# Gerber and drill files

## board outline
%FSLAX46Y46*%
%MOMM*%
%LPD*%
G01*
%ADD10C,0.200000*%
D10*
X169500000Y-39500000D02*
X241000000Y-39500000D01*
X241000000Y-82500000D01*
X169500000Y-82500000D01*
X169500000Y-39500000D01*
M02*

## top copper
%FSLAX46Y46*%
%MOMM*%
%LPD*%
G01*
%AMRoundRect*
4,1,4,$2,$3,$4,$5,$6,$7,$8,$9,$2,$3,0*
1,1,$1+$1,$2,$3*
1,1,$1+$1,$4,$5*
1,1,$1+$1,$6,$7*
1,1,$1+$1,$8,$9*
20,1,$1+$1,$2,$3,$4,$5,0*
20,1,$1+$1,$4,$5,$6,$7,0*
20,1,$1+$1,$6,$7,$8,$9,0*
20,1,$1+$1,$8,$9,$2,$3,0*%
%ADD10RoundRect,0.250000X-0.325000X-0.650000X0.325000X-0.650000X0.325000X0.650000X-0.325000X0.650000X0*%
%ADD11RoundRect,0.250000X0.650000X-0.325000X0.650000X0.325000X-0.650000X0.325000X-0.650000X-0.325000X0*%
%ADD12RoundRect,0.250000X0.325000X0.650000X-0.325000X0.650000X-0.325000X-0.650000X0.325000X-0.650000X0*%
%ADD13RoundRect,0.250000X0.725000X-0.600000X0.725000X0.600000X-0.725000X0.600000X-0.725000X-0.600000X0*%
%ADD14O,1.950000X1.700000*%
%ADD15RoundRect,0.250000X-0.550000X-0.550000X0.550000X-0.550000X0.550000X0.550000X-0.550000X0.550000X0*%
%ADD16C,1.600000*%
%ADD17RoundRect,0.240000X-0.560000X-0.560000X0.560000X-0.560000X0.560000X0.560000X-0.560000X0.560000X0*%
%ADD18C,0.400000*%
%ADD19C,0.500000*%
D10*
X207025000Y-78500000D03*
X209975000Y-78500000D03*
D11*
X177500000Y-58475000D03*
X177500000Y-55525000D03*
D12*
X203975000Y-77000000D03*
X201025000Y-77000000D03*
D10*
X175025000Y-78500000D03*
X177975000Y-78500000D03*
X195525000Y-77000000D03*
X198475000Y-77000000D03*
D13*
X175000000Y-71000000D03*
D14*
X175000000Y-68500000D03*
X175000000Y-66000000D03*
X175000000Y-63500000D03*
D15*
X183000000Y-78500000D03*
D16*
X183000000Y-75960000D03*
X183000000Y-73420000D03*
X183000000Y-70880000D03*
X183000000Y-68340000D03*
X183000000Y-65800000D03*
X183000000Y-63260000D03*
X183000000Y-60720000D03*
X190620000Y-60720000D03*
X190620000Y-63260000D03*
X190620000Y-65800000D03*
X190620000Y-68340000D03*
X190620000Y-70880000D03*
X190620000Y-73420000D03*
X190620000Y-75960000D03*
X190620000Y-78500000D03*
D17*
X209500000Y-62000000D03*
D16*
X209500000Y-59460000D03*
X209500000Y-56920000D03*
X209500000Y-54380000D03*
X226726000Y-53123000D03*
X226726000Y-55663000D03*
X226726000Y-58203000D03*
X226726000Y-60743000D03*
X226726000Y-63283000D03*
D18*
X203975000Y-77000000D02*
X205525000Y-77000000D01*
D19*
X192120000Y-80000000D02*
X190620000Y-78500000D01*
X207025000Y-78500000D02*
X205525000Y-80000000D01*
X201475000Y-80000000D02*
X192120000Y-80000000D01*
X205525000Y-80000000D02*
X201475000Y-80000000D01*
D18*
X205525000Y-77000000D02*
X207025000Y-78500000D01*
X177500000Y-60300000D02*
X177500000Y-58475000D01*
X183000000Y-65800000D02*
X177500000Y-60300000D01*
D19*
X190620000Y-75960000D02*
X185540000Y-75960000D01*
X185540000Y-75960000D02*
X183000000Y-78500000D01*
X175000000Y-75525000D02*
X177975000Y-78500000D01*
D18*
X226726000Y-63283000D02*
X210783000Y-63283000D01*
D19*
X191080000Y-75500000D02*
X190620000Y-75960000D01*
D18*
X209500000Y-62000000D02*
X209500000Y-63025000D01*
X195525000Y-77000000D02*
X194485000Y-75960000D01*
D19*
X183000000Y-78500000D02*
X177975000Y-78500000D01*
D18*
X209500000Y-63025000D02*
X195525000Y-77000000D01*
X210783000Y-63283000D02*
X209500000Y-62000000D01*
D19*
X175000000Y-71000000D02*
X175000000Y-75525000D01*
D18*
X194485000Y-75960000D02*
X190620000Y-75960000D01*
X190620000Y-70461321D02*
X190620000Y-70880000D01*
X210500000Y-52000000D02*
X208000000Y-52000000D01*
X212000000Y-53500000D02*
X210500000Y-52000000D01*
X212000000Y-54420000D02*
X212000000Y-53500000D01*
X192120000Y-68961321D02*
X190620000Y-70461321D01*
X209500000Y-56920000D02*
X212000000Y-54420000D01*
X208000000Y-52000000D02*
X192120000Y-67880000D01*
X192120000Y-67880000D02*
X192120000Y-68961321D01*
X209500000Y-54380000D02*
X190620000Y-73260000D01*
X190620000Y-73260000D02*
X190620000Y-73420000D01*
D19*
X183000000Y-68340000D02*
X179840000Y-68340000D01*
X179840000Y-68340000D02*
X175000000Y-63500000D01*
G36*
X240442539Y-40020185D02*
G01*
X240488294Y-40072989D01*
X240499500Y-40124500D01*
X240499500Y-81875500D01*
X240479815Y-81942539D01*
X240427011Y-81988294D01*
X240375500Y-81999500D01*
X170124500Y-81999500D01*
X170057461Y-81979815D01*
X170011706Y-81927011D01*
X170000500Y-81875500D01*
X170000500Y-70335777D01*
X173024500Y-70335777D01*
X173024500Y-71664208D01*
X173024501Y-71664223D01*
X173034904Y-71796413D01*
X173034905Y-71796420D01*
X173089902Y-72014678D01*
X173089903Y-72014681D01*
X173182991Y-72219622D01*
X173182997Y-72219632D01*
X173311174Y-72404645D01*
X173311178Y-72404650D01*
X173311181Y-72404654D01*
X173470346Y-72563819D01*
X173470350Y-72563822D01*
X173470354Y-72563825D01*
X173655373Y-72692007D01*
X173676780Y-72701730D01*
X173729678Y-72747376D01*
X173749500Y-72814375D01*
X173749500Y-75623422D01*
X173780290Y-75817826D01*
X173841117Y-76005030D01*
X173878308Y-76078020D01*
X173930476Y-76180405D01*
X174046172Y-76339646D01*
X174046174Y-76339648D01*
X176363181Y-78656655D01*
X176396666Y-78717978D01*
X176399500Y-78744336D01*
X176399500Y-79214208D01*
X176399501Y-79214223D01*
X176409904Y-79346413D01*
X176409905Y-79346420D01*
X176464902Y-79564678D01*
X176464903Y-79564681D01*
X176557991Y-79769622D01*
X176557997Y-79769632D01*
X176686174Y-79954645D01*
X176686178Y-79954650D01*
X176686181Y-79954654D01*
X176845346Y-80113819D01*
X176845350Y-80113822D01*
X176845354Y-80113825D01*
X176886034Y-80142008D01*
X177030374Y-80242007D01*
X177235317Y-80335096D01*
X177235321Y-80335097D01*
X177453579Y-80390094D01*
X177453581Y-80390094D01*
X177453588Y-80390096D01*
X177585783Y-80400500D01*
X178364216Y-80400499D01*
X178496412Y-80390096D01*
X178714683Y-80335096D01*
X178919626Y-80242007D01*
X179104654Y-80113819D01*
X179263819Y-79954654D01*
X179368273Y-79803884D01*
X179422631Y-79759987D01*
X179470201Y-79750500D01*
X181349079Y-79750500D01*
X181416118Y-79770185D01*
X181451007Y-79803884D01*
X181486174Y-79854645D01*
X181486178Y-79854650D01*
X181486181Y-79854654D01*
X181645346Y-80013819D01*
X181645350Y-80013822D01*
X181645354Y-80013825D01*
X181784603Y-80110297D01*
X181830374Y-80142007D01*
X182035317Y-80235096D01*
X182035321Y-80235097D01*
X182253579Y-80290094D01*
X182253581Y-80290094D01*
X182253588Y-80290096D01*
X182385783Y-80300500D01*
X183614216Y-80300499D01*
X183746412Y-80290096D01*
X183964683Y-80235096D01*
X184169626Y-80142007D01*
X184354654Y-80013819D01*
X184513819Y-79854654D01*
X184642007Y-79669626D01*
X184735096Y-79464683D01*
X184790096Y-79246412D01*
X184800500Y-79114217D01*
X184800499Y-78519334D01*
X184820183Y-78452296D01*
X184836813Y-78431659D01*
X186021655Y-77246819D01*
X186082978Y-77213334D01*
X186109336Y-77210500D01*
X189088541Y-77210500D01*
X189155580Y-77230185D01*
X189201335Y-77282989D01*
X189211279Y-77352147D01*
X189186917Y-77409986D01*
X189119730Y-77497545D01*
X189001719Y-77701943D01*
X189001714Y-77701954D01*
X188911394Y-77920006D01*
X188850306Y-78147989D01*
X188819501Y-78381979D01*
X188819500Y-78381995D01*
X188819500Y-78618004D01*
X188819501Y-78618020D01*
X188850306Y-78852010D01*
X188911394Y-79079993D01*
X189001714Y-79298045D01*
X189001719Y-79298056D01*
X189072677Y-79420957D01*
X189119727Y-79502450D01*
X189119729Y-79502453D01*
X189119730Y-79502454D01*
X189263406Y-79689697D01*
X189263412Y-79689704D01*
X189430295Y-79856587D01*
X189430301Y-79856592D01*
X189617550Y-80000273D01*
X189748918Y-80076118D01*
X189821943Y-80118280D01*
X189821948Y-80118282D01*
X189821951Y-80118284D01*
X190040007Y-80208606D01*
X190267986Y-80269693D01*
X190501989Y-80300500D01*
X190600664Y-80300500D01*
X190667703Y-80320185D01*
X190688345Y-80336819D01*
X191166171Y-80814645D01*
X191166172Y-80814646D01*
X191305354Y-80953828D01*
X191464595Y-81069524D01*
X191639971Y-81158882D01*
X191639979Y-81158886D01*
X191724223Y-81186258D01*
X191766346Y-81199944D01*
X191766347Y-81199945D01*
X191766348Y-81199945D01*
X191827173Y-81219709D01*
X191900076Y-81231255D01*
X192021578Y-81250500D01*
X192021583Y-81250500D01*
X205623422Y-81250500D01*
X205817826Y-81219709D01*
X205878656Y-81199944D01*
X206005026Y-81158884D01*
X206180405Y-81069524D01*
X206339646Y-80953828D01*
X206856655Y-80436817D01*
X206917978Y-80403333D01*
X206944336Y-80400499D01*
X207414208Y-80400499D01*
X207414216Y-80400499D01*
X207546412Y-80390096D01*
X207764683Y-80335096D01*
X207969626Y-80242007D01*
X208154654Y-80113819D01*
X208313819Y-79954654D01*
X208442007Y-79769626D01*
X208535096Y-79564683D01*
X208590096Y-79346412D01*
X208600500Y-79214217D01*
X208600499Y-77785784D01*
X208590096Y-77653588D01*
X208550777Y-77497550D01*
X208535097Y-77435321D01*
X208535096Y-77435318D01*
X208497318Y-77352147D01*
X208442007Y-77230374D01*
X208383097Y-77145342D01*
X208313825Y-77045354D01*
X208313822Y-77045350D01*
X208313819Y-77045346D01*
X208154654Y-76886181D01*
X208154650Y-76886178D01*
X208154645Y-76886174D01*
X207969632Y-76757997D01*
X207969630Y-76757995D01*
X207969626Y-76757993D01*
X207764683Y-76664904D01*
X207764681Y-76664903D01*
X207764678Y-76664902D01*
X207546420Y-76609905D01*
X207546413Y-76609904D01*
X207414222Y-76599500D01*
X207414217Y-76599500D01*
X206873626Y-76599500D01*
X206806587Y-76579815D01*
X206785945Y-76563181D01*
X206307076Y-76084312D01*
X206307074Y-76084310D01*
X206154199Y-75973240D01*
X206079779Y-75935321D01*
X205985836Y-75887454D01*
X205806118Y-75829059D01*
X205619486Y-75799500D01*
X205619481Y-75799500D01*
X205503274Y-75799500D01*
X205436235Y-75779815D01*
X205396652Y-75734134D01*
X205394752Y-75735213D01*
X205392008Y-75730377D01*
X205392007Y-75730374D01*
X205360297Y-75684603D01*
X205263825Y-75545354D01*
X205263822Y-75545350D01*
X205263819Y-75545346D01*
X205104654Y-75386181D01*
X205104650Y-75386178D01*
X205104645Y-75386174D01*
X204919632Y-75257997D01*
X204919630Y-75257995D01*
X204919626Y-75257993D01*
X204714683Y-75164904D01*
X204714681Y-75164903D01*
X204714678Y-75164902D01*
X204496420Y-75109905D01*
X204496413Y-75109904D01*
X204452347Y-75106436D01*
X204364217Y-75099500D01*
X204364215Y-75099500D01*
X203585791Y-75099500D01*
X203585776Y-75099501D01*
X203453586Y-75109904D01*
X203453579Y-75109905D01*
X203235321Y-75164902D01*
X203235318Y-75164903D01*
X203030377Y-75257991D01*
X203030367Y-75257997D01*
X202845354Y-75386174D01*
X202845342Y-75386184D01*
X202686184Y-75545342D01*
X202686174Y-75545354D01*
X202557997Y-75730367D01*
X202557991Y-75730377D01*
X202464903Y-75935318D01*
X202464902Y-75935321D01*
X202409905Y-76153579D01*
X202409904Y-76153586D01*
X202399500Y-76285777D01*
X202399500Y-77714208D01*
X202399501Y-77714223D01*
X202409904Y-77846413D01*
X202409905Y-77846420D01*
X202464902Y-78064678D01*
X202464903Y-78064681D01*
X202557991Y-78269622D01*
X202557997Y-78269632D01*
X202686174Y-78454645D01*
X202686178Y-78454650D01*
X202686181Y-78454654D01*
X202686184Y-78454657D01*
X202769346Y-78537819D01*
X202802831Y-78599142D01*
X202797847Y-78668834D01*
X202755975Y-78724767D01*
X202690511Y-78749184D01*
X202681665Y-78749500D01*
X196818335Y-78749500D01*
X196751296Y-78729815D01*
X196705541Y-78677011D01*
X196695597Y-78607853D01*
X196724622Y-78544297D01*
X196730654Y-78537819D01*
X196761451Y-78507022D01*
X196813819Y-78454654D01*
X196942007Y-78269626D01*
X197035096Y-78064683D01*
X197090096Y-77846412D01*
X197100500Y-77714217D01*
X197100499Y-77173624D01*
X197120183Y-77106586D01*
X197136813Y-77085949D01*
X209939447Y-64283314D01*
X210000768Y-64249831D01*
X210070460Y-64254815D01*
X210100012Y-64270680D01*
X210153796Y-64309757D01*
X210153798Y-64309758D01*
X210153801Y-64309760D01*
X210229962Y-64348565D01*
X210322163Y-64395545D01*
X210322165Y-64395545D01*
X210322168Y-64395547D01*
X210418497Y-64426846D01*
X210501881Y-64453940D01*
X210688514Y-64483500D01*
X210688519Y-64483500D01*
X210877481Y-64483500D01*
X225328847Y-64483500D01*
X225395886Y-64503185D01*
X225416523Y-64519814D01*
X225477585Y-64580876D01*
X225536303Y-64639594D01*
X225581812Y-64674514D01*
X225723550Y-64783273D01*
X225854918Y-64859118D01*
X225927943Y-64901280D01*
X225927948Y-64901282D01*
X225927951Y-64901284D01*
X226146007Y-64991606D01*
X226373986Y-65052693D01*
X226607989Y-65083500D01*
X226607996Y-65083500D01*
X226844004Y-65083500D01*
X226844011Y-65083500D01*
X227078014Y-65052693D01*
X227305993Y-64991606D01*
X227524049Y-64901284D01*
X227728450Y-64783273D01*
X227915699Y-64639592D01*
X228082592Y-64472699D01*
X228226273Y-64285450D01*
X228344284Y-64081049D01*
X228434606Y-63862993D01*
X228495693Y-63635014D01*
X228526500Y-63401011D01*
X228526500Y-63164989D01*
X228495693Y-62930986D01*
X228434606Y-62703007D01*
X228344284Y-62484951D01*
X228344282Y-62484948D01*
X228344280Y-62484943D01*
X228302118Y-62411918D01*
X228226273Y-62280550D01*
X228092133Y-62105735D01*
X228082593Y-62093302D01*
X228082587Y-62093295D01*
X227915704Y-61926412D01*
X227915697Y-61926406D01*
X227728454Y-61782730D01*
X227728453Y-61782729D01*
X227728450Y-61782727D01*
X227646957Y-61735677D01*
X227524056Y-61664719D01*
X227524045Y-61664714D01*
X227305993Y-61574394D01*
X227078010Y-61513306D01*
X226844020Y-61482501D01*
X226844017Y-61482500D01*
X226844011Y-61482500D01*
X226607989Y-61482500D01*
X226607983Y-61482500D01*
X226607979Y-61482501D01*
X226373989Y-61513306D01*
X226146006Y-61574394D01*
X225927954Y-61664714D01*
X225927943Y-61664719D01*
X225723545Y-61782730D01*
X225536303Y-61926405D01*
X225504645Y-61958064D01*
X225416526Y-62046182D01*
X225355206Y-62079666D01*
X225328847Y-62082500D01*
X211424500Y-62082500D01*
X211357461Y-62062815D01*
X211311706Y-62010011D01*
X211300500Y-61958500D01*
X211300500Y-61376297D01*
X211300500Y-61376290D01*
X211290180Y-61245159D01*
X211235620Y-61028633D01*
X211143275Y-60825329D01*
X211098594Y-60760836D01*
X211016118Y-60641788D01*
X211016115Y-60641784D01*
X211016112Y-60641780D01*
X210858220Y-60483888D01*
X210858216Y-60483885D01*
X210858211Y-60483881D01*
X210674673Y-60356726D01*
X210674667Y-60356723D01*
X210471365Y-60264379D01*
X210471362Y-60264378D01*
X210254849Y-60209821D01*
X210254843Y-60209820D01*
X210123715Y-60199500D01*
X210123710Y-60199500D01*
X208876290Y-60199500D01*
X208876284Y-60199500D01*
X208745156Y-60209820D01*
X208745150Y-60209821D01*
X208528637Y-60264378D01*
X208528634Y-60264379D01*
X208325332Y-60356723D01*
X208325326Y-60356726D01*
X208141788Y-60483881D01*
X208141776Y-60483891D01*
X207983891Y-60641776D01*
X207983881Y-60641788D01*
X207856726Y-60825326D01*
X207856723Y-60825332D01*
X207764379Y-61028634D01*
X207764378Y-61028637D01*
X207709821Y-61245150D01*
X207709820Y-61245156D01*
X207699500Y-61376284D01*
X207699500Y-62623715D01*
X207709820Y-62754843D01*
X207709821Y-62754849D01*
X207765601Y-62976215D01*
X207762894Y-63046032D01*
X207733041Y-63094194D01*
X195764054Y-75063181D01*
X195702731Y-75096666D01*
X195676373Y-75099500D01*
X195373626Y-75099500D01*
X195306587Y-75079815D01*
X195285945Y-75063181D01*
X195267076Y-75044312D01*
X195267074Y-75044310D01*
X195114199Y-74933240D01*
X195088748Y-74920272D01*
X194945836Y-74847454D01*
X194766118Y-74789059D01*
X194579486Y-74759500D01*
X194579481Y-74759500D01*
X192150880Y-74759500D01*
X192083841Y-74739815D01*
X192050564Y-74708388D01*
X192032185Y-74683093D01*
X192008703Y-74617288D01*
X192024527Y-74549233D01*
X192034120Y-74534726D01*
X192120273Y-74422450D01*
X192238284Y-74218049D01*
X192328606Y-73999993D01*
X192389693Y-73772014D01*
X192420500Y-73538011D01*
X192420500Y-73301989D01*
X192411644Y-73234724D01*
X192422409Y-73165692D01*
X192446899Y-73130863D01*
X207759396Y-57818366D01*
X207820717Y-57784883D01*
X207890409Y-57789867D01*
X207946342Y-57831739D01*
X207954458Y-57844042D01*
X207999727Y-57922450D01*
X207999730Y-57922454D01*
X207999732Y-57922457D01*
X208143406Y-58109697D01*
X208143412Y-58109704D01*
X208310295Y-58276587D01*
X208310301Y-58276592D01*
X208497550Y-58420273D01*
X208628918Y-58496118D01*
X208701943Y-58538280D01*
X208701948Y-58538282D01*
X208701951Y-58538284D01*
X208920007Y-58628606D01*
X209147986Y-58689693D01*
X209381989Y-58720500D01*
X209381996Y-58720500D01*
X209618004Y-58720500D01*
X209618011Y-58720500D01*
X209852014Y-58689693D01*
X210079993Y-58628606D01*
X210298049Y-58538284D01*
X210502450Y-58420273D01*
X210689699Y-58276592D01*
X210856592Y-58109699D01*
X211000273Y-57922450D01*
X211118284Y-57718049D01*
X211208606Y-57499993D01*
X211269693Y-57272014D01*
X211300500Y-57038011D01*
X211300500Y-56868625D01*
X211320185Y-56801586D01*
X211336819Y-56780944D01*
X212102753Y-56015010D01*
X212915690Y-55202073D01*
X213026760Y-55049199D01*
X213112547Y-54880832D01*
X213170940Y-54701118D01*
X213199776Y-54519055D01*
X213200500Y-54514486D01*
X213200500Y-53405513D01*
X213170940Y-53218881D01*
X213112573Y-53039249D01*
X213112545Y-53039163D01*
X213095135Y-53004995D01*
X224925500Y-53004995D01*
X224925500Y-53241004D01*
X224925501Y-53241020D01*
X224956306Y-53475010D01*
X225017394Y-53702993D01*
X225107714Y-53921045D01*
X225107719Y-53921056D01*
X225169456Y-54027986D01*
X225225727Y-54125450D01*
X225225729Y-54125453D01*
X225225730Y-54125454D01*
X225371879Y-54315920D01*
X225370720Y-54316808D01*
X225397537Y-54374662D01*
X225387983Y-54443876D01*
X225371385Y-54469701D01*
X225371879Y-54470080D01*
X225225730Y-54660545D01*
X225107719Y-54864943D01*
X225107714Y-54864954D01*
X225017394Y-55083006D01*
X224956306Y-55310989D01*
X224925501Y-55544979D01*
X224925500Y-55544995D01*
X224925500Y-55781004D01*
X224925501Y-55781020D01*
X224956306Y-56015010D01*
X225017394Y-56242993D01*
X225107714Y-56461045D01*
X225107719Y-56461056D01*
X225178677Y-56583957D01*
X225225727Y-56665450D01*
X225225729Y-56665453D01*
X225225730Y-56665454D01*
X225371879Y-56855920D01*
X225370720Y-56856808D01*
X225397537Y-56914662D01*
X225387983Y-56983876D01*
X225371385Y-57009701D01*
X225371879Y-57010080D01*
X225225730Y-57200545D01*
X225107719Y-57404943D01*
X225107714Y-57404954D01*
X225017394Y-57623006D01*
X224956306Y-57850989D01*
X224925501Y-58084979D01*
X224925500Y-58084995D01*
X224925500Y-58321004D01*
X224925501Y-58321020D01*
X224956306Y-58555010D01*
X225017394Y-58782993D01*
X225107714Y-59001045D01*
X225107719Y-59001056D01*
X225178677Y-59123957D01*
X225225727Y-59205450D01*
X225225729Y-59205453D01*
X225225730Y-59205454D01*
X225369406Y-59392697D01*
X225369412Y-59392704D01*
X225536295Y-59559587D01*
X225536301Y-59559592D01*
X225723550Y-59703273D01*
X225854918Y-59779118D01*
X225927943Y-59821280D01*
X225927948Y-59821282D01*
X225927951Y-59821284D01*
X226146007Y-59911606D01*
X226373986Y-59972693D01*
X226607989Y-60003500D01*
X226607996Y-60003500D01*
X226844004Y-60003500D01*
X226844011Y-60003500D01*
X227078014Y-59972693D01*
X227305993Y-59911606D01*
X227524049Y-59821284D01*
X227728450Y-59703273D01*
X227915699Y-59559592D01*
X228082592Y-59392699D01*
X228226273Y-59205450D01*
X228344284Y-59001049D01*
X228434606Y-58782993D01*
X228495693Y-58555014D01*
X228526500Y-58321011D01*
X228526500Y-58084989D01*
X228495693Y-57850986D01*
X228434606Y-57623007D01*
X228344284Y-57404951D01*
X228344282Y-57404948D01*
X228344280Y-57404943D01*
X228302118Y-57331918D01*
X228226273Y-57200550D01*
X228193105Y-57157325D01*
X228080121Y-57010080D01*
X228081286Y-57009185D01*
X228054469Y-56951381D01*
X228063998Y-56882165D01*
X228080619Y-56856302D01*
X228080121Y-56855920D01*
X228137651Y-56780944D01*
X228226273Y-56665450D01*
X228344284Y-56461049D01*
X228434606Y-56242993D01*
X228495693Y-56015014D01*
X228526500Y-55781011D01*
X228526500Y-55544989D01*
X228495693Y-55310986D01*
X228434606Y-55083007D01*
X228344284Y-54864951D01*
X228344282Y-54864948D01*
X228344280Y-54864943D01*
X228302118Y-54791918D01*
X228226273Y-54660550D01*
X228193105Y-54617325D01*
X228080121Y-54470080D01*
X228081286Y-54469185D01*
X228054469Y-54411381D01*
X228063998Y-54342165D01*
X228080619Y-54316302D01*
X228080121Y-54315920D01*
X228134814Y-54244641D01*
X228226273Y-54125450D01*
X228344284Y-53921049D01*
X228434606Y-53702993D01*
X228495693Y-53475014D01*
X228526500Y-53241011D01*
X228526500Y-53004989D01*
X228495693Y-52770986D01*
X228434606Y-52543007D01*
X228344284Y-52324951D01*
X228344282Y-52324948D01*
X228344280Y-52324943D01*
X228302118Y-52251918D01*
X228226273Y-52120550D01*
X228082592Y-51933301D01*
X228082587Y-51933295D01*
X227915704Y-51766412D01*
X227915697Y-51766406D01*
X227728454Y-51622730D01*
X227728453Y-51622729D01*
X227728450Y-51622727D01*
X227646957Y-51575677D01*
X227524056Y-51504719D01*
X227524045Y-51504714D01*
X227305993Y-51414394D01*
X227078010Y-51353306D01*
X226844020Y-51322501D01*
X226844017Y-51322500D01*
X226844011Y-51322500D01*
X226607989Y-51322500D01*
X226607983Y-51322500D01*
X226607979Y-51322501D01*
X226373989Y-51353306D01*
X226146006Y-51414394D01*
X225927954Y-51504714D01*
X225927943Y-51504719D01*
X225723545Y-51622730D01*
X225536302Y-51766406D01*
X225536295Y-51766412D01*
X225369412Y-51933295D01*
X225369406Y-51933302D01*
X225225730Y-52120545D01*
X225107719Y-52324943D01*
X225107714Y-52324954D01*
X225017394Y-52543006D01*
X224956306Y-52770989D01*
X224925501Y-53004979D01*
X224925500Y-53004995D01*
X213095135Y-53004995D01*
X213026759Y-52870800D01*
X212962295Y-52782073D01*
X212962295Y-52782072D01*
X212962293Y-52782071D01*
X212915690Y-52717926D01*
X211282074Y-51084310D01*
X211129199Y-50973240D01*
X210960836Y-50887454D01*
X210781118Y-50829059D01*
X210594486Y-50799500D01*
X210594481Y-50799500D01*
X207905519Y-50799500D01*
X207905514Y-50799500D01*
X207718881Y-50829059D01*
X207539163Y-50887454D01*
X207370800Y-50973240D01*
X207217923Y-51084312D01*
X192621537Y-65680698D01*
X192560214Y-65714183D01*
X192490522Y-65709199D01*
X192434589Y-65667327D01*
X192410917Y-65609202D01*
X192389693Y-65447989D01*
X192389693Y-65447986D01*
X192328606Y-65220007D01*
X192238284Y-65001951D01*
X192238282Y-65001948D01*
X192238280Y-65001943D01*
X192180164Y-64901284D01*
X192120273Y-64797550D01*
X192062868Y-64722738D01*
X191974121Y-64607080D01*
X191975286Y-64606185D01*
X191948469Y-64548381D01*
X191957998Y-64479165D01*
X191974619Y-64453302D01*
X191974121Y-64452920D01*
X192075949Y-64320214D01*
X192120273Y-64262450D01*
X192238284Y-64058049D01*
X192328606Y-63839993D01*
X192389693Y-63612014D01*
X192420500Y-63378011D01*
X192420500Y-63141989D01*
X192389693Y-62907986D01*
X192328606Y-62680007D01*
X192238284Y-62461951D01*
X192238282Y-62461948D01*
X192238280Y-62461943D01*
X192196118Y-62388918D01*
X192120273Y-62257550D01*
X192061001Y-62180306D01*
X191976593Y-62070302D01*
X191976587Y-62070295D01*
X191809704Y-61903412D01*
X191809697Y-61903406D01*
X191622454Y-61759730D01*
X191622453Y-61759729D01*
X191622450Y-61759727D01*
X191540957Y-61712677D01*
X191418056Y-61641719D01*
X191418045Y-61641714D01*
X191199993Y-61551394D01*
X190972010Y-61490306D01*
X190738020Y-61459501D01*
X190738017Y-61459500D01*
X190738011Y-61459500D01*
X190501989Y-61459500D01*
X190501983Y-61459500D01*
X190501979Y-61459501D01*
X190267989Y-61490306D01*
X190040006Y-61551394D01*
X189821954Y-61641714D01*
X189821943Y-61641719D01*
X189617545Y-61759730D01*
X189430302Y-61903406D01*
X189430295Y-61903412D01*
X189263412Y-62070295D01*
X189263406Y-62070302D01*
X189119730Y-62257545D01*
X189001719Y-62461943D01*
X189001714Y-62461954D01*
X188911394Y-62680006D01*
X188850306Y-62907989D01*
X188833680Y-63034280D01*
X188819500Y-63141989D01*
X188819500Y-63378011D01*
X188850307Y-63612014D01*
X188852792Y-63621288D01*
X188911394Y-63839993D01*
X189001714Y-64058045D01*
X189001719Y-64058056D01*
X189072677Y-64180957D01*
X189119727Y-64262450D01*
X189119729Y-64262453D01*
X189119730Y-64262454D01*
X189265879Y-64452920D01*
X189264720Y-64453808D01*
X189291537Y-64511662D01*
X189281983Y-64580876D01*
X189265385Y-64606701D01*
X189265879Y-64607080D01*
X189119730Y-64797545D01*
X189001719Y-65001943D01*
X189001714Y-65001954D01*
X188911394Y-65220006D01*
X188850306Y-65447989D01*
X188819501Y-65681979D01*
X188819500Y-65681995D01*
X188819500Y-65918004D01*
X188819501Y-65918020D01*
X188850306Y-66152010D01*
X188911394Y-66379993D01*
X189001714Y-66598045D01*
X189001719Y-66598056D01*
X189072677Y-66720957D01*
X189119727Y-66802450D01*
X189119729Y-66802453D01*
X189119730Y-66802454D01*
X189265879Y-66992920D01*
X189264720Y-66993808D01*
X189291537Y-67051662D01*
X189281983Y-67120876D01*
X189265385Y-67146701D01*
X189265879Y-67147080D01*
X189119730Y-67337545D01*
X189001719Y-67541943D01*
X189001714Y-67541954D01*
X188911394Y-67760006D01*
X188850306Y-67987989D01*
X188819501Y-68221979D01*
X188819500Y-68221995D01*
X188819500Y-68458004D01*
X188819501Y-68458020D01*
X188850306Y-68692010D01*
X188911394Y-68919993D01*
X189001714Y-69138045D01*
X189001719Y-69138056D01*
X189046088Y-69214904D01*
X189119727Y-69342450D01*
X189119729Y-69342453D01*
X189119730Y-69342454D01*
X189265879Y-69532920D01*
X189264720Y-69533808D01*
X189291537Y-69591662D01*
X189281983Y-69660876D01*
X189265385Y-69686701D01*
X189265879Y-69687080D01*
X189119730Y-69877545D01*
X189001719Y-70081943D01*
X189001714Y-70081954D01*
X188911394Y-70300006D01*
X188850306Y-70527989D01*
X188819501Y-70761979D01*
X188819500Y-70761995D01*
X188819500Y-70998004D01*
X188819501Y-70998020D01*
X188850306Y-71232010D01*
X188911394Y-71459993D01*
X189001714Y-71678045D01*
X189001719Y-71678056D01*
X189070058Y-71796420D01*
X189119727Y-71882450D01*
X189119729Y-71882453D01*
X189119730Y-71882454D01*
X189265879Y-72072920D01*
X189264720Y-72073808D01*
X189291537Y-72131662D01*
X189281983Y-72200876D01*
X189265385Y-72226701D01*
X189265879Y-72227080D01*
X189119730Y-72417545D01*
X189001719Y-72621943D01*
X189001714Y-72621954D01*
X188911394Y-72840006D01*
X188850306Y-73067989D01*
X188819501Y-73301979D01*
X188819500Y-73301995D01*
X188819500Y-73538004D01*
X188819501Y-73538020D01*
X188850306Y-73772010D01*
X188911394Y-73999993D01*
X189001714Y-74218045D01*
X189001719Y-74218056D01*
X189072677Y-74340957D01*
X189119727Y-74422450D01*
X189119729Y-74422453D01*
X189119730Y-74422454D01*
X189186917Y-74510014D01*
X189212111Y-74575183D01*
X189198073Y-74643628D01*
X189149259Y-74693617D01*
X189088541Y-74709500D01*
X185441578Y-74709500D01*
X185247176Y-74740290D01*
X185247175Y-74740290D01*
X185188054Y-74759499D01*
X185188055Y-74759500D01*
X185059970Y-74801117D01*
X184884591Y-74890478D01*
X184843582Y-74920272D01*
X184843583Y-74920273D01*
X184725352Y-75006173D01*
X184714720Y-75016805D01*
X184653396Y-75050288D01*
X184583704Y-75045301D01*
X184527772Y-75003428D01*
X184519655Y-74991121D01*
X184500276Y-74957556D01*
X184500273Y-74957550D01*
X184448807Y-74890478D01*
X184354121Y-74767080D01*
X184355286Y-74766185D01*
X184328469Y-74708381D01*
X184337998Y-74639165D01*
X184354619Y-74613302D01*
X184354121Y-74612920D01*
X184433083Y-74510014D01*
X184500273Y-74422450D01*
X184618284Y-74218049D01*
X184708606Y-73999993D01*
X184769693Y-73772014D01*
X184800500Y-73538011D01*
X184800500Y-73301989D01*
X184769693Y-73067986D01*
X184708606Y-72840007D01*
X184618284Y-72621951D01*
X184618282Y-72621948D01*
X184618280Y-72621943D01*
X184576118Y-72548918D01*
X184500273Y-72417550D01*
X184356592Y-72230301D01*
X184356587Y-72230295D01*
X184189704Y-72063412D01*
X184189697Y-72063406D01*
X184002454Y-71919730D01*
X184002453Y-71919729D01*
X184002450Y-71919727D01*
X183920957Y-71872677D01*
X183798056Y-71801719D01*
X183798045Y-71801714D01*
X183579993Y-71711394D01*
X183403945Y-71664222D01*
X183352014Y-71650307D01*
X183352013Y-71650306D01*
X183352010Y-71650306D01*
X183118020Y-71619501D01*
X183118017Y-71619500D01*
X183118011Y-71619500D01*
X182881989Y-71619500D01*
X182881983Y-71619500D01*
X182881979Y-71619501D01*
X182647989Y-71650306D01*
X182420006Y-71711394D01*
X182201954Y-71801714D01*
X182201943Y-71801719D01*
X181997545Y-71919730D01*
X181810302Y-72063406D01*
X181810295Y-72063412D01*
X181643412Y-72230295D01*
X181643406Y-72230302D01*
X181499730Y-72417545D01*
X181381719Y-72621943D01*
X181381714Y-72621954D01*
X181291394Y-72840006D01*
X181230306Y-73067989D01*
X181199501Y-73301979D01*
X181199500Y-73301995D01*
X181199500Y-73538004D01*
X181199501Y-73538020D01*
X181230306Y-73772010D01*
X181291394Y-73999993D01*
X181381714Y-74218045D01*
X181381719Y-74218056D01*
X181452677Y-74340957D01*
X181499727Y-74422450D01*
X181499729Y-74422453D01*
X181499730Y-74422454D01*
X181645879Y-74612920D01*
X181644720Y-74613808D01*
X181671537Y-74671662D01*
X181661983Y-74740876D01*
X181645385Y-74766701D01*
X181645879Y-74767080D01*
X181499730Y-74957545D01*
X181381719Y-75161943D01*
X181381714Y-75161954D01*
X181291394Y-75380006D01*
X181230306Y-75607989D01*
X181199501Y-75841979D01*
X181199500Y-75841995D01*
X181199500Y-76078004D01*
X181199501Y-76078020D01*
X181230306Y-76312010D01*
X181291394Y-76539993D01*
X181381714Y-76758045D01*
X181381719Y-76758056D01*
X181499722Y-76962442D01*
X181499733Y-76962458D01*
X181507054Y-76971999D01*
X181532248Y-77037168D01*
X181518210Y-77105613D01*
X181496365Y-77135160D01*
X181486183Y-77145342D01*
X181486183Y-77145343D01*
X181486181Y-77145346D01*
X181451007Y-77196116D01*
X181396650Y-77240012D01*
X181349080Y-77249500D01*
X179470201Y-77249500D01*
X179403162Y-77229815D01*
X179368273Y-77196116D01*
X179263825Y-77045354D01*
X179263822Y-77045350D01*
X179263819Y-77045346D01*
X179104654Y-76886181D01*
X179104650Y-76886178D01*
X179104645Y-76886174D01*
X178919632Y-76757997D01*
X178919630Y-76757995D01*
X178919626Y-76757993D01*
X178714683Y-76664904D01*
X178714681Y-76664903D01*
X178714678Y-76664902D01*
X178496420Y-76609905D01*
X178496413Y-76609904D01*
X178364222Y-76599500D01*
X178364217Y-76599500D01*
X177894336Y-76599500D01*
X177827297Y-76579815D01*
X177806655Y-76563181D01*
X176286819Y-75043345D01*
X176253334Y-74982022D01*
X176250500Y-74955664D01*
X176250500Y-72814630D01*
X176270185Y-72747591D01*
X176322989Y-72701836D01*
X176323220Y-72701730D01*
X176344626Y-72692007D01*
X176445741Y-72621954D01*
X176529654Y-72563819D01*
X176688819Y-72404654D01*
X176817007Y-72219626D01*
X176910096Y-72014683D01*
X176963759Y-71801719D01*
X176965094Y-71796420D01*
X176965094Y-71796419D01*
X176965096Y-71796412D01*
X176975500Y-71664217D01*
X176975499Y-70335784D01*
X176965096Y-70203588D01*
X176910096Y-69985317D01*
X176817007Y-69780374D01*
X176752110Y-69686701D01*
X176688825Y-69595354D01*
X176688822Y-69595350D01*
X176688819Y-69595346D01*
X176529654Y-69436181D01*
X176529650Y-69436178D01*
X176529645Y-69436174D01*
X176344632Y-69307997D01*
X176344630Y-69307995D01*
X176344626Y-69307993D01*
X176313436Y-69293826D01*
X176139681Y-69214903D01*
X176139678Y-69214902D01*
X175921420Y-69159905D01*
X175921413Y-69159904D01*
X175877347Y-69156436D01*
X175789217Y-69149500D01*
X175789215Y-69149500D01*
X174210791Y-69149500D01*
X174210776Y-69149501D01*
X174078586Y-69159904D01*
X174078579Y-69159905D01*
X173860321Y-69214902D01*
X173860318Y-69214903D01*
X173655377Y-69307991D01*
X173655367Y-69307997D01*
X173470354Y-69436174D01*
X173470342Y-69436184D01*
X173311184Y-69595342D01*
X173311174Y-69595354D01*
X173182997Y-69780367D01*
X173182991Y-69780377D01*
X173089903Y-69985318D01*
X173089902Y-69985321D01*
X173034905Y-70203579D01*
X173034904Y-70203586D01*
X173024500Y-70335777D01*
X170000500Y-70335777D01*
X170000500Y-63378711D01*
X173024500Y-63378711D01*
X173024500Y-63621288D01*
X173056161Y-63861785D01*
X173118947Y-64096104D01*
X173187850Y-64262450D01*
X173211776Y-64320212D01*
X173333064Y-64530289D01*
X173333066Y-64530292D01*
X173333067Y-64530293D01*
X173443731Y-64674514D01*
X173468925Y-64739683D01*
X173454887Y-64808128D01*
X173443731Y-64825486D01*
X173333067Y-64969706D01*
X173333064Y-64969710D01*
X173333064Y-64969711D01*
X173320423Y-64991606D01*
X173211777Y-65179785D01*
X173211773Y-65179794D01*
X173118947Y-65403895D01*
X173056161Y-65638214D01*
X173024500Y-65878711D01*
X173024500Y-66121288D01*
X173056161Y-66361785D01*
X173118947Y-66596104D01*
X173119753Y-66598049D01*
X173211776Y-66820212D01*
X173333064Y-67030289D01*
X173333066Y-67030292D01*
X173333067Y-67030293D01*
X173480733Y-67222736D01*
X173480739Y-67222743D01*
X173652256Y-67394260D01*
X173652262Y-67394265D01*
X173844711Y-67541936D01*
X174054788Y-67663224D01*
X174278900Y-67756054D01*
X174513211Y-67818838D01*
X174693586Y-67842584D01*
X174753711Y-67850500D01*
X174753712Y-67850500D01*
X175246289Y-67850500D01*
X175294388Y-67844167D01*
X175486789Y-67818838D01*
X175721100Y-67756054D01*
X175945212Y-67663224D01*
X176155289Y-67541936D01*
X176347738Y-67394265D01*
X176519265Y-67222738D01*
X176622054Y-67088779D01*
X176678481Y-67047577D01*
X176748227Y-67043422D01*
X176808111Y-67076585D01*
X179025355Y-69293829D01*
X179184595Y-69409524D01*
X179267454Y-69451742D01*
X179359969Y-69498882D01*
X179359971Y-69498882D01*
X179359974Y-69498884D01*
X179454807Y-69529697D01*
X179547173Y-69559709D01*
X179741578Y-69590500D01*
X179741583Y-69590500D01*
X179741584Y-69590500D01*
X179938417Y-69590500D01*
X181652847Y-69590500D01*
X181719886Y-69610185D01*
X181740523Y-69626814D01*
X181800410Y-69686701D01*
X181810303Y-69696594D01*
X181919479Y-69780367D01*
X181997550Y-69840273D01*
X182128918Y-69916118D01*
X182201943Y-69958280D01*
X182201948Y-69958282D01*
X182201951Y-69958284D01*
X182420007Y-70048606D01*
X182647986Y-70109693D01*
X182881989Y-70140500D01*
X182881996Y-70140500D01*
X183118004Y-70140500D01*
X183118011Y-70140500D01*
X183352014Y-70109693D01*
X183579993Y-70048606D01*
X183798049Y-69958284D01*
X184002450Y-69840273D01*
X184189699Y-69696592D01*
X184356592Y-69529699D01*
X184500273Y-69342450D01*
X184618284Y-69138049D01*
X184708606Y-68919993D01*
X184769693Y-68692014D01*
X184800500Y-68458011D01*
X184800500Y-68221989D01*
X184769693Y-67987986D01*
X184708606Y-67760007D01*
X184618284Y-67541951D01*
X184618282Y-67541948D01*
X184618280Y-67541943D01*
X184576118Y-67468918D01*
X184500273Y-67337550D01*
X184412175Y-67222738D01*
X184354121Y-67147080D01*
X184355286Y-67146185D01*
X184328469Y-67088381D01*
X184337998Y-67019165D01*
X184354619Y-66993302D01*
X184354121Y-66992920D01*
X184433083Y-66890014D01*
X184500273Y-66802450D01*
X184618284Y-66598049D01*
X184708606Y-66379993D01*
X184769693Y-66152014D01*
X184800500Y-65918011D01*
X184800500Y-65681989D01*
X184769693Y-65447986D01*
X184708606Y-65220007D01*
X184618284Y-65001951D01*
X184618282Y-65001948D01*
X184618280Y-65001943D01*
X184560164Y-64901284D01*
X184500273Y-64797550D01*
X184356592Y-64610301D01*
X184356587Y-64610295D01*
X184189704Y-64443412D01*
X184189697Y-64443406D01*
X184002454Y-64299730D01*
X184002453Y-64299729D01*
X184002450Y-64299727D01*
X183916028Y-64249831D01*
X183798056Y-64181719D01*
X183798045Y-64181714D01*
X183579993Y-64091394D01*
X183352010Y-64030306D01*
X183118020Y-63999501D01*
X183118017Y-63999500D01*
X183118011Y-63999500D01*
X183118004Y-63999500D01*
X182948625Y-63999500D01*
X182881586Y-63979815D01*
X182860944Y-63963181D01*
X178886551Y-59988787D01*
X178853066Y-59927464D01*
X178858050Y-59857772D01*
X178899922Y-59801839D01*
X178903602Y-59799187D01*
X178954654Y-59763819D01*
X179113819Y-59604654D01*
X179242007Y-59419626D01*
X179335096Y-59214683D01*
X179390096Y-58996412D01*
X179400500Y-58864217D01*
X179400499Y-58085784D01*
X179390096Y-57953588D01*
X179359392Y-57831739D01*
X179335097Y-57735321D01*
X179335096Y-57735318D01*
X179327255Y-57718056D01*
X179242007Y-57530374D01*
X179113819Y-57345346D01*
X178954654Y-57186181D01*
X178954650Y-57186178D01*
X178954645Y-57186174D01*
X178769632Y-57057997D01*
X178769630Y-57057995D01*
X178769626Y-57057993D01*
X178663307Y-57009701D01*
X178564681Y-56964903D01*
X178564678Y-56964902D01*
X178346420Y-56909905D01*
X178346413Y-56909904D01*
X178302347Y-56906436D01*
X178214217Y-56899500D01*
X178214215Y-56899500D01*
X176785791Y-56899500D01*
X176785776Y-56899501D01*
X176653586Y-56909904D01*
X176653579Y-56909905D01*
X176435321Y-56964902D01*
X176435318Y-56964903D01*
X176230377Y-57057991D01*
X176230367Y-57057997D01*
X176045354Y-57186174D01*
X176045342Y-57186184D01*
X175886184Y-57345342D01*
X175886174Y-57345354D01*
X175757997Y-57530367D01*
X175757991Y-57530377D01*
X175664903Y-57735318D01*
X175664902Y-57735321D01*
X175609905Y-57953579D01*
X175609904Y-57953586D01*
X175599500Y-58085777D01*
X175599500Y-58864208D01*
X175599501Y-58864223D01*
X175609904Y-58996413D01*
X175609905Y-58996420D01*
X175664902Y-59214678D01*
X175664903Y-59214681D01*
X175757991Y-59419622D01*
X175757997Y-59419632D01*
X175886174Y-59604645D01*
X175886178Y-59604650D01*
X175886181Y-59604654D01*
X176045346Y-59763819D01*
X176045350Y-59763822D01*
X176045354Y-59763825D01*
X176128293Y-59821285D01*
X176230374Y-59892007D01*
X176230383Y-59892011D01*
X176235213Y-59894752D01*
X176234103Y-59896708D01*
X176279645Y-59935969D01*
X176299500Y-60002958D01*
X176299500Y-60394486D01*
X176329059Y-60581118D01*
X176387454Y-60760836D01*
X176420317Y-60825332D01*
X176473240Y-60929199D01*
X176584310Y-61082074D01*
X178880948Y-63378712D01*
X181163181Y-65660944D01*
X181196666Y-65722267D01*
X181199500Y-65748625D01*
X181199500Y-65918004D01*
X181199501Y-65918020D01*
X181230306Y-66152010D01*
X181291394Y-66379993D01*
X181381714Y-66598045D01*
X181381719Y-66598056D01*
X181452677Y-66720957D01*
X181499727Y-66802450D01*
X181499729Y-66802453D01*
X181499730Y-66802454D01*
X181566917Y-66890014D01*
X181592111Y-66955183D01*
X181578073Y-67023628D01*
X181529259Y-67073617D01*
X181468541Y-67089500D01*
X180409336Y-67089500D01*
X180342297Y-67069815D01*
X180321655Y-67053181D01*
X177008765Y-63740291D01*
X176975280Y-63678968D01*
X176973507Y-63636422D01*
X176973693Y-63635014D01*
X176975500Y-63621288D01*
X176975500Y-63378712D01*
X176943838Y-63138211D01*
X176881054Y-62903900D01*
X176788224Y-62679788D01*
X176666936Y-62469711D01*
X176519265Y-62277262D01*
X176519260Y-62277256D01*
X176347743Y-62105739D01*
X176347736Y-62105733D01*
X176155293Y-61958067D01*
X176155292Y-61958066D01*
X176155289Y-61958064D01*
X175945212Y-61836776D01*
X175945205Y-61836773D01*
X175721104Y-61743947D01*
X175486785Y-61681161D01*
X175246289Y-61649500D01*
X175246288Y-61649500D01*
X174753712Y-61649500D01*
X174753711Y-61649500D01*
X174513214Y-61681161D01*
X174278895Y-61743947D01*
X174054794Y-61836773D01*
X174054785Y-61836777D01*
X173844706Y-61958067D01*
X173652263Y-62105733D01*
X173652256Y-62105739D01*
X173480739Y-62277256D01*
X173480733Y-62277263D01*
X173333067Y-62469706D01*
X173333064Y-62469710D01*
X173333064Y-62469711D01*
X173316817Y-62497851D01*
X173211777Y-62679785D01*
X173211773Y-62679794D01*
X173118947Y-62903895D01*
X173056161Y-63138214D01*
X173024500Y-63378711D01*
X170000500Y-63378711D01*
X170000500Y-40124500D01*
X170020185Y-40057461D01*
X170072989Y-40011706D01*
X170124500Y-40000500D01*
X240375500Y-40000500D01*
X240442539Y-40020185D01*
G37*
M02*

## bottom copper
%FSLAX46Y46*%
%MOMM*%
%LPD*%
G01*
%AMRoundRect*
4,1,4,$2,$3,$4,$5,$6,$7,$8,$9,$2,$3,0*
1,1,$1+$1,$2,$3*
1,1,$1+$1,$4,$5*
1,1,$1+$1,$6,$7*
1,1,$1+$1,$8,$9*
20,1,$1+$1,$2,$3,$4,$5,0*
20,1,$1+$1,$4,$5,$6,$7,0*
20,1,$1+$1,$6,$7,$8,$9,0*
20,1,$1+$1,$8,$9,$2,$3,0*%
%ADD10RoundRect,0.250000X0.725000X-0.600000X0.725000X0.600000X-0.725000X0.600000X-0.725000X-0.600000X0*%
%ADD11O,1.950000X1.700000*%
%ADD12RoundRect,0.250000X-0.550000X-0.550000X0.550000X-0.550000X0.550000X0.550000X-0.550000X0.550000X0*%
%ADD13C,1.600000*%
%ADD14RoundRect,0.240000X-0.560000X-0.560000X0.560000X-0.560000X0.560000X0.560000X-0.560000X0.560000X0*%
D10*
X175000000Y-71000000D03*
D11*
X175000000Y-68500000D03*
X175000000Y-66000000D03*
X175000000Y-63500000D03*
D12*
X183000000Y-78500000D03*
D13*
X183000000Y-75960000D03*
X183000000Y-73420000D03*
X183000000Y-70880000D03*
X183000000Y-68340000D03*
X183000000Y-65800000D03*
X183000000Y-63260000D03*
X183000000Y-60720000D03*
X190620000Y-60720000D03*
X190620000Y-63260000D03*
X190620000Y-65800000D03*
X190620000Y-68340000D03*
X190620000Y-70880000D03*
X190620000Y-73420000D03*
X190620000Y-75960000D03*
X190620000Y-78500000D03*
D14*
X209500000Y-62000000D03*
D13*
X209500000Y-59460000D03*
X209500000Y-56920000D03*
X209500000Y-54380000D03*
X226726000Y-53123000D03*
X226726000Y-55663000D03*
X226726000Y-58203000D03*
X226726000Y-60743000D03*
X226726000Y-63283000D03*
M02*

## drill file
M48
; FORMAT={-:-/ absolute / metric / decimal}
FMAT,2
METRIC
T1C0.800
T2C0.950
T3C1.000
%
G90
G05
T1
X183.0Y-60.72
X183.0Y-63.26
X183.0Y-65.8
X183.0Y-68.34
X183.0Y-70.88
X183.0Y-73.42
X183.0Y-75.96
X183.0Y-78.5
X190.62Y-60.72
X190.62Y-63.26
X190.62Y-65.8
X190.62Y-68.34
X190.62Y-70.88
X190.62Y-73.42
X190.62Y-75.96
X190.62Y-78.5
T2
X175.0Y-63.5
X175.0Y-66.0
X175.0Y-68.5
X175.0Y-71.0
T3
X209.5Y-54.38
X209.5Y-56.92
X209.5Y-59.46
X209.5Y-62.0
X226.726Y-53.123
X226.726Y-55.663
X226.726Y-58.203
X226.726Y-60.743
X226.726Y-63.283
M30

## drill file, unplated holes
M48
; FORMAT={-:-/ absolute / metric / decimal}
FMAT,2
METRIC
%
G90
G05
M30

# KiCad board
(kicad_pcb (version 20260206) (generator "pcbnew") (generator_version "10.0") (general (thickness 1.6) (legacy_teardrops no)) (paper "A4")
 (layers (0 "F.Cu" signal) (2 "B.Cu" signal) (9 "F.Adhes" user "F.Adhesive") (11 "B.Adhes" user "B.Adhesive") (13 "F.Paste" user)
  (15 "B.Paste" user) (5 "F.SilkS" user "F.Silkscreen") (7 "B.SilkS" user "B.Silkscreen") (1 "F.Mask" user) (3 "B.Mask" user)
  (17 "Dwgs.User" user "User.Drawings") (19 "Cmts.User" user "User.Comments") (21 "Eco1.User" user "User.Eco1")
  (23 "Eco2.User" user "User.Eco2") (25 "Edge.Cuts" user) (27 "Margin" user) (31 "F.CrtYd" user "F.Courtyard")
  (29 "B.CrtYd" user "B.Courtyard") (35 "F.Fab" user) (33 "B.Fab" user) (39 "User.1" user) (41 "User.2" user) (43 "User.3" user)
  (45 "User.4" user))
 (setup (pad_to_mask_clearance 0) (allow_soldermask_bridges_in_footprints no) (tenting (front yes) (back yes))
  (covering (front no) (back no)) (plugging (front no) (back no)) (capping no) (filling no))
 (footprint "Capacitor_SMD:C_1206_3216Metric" (layer "F.Cu") (at 208.5 78.5)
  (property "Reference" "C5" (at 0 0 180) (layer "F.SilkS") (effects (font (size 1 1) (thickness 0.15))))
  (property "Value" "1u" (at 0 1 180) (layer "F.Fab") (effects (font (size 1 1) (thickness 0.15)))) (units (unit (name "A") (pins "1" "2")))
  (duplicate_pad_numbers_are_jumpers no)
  (pad "1" smd roundrect (at -1.475 0) (size 1.15 1.8) (layers "F.Cu" "F.Mask" "F.Paste") (roundrect_rratio 0.217391)
   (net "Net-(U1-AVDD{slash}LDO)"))
  (pad "2" smd roundrect (at 1.475 0) (size 1.15 1.8) (layers "F.Cu" "F.Mask" "F.Paste") (roundrect_rratio 0.217391) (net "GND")))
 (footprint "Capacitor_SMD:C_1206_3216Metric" (layer "F.Cu") (at 177.5 57 90)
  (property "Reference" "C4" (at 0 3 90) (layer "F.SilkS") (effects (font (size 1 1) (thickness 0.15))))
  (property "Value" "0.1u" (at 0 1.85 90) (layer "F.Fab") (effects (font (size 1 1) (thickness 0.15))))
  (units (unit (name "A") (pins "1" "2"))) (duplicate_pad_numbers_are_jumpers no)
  (pad "1" smd roundrect (at -1.475 0 90) (size 1.15 1.8) (layers "F.Cu" "F.Mask" "F.Paste") (roundrect_rratio 0.217391)
   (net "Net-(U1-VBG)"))
  (pad "2" smd roundrect (at 1.475 0 90) (size 1.15 1.8) (layers "F.Cu" "F.Mask" "F.Paste") (roundrect_rratio 0.217391) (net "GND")))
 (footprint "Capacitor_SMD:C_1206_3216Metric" (layer "F.Cu") (at 202.5 77 180)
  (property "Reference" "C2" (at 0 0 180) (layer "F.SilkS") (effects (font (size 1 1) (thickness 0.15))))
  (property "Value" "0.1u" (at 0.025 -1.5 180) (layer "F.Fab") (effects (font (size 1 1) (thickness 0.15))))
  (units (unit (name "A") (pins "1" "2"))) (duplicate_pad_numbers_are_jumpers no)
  (pad "1" smd roundrect (at -1.475 0 180) (size 1.15 1.8) (layers "F.Cu" "F.Mask" "F.Paste") (roundrect_rratio 0.217391)
   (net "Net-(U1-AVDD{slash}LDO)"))
  (pad "2" smd roundrect (at 1.475 0 180) (size 1.15 1.8) (layers "F.Cu" "F.Mask" "F.Paste") (roundrect_rratio 0.217391) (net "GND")))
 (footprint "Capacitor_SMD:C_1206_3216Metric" (layer "F.Cu") (at 176.5 78.5)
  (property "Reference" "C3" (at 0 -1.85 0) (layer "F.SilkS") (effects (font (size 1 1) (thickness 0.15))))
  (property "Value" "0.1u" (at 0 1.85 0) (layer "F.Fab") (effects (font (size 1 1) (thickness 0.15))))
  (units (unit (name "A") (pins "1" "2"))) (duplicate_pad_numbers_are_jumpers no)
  (pad "1" smd roundrect (at -1.475 0) (size 1.15 1.8) (layers "F.Cu" "F.Mask" "F.Paste") (roundrect_rratio 0.217391) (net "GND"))
  (pad "2" smd roundrect (at 1.475 0) (size 1.15 1.8) (layers "F.Cu" "F.Mask" "F.Paste") (roundrect_rratio 0.217391) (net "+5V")))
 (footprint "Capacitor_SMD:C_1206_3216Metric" (layer "F.Cu") (at 197 77)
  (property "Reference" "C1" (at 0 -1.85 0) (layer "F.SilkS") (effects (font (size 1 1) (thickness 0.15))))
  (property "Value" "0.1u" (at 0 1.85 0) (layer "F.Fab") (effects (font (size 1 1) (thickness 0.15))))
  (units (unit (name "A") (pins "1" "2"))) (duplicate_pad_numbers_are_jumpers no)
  (pad "1" smd roundrect (at -1.475 0) (size 1.15 1.8) (layers "F.Cu" "F.Mask" "F.Paste") (roundrect_rratio 0.217391) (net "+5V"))
  (pad "2" smd roundrect (at 1.475 0) (size 1.15 1.8) (layers "F.Cu" "F.Mask" "F.Paste") (roundrect_rratio 0.217391) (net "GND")))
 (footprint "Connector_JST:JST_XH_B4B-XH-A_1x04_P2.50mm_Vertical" (layer "B.Cu") (at 175 71 90)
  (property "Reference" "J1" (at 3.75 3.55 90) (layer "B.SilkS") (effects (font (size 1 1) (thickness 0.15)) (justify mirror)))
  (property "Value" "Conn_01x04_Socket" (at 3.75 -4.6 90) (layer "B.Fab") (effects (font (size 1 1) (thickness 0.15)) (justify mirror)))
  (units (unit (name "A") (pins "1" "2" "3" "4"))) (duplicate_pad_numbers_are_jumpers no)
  (pad "1" thru_hole roundrect (at 0 0 90) (size 1.7 1.95) (drill 0.95) (layers "*.Cu" "*.Mask") (remove_unused_layers no)
   (roundrect_rratio 0.147059) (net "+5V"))
  (pad "2" thru_hole oval (at 2.5 0 90) (size 1.7 1.95) (drill 0.95) (layers "*.Cu" "*.Mask") (remove_unused_layers no) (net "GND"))
  (pad "3" thru_hole oval (at 5 0 90) (size 1.7 1.95) (drill 0.95) (layers "*.Cu" "*.Mask") (remove_unused_layers no)
   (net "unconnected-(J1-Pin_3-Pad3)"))
  (pad "4" thru_hole oval (at 7.5 0 90) (size 1.7 1.95) (drill 0.95) (layers "*.Cu" "*.Mask") (remove_unused_layers no) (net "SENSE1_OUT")))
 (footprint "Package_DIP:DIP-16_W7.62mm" (layer "B.Cu") (at 183 78.5)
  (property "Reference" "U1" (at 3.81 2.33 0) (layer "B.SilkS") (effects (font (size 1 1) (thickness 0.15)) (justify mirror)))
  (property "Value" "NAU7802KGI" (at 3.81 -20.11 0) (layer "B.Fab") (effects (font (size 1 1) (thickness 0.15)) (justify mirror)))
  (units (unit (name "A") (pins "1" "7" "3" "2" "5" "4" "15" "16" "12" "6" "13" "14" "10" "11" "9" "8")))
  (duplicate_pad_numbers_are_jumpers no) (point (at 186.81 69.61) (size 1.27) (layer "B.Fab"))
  (pad "1" thru_hole roundrect (at 0 0) (size 1.6 1.6) (drill 0.8) (layers "*.Cu" "*.Mask") (remove_unused_layers no)
   (roundrect_rratio 0.15625) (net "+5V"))
  (pad "2" thru_hole circle (at 0 -2.54) (size 1.6 1.6) (drill 0.8) (layers "*.Cu" "*.Mask") (remove_unused_layers no)
   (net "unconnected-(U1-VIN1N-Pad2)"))
  (pad "3" thru_hole circle (at 0 -5.08) (size 1.6 1.6) (drill 0.8) (layers "*.Cu" "*.Mask") (remove_unused_layers no)
   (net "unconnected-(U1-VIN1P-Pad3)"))
  (pad "4" thru_hole circle (at 0 -7.62) (size 1.6 1.6) (drill 0.8) (layers "*.Cu" "*.Mask") (remove_unused_layers no) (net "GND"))
  (pad "5" thru_hole circle (at 0 -10.16) (size 1.6 1.6) (drill 0.8) (layers "*.Cu" "*.Mask") (remove_unused_layers no) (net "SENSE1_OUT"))
  (pad "6" thru_hole circle (at 0 -12.7) (size 1.6 1.6) (drill 0.8) (layers "*.Cu" "*.Mask") (remove_unused_layers no) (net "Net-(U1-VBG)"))
  (pad "7" thru_hole circle (at 0 -15.24) (size 1.6 1.6) (drill 0.8) (layers "*.Cu" "*.Mask") (remove_unused_layers no) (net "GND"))
  (pad "8" thru_hole circle (at 0 -17.78) (size 1.6 1.6) (drill 0.8) (layers "*.Cu" "*.Mask") (remove_unused_layers no) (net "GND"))
  (pad "9" thru_hole circle (at 7.62 -17.78) (size 1.6 1.6) (drill 0.8) (layers "*.Cu" "*.Mask") (remove_unused_layers no) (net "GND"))
  (pad "10" thru_hole circle (at 7.62 -15.24) (size 1.6 1.6) (drill 0.8) (layers "*.Cu" "*.Mask") (remove_unused_layers no)
   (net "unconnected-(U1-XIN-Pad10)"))
  (pad "11" thru_hole circle (at 7.62 -12.7) (size 1.6 1.6) (drill 0.8) (layers "*.Cu" "*.Mask") (remove_unused_layers no)
   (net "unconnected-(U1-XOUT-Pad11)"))
  (pad "12" thru_hole circle (at 7.62 -10.16) (size 1.6 1.6) (drill 0.8) (layers "*.Cu" "*.Mask") (remove_unused_layers no)
   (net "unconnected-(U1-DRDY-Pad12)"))
  (pad "13" thru_hole circle (at 7.62 -7.62) (size 1.6 1.6) (drill 0.8) (layers "*.Cu" "*.Mask") (remove_unused_layers no) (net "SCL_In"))
  (pad "14" thru_hole circle (at 7.62 -5.08) (size 1.6 1.6) (drill 0.8) (layers "*.Cu" "*.Mask") (remove_unused_layers no) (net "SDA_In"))
  (pad "15" thru_hole circle (at 7.62 -2.54) (size 1.6 1.6) (drill 0.8) (layers "*.Cu" "*.Mask") (remove_unused_layers no) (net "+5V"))
  (pad "16" thru_hole circle (at 7.62 0) (size 1.6 1.6) (drill 0.8) (layers "*.Cu" "*.Mask") (remove_unused_layers no)
   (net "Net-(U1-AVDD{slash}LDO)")))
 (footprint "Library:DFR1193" (layer "B.Cu") (at 209.5 62)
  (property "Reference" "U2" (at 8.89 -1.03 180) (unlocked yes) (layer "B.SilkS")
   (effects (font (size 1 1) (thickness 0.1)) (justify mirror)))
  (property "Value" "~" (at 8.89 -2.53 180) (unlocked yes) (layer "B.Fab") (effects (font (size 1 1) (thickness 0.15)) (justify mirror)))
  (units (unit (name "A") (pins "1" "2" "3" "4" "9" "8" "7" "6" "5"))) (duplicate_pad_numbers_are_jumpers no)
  (pad "1" thru_hole roundrect (at 0 0) (size 1.6 1.6) (drill 1) (layers "*.Cu" "*.Mask") (remove_unused_layers no) (roundrect_rratio 0.15)
   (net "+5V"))
  (pad "2" thru_hole circle (at 0 -2.54) (size 1.6 1.6) (drill 1) (layers "*.Cu" "*.Mask") (remove_unused_layers no) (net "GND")
   (thermal_bridge_angle 90))
  (pad "3" thru_hole circle (at 0 -5.08) (size 1.6 1.6) (drill 1) (layers "*.Cu" "*.Mask") (remove_unused_layers no) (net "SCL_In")
   (thermal_bridge_angle 90))
  (pad "4" thru_hole circle (at 0 -7.62) (size 1.6 1.6) (drill 1) (layers "*.Cu" "*.Mask") (remove_unused_layers no) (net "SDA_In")
   (thermal_bridge_angle 90))
  (pad "5" thru_hole circle (at 17.226 -8.877) (size 1.6 1.6) (drill 1) (layers "*.Cu" "*.Mask") (remove_unused_layers no)
   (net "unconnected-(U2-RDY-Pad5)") (thermal_bridge_angle 90))
  (pad "6" thru_hole circle (at 17.226 -6.337) (size 1.6 1.6) (drill 1) (layers "*.Cu" "*.Mask") (remove_unused_layers no)
   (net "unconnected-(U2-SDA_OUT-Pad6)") (thermal_bridge_angle 90))
  (pad "7" thru_hole circle (at 17.226 -3.797) (size 1.6 1.6) (drill 1) (layers "*.Cu" "*.Mask") (remove_unused_layers no)
   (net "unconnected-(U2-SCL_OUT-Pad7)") (thermal_bridge_angle 90))
  (pad "8" thru_hole circle (at 17.226 -1.257) (size 1.6 1.6) (drill 1) (layers "*.Cu" "*.Mask") (remove_unused_layers no) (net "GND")
   (thermal_bridge_angle 90))
  (pad "9" thru_hole circle (at 17.226 1.283) (size 1.6 1.6) (drill 1) (layers "*.Cu" "*.Mask") (remove_unused_layers no) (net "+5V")
   (thermal_bridge_angle 90)))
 (gr_rect (start 169.5 39.5) (end 241 82.5) (stroke (width 0.2) (type default)) (fill no) (layer "Edge.Cuts"))
 (segment (start 203.975 77) (end 205.525 77) (width 0.4) (layer "F.Cu") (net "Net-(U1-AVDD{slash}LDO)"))
 (segment (start 192.12 80) (end 190.62 78.5) (width 0.5) (layer "F.Cu") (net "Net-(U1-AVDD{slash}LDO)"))
 (segment (start 207.025 78.5) (end 205.525 80) (width 0.5) (layer "F.Cu") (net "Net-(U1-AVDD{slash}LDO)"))
 (segment (start 201.475 80) (end 192.12 80) (width 0.5) (layer "F.Cu") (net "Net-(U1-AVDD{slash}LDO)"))
 (segment (start 205.525 80) (end 201.475 80) (width 0.5) (layer "F.Cu") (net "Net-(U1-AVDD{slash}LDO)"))
 (segment (start 205.525 77) (end 207.025 78.5) (width 0.4) (layer "F.Cu") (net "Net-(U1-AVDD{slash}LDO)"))
 (segment (start 177.5 60.3) (end 177.5 58.475) (width 0.4) (layer "F.Cu") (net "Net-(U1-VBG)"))
 (segment (start 183 65.8) (end 177.5 60.3) (width 0.4) (layer "F.Cu") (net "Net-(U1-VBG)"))
 (segment (start 190.62 75.96) (end 185.54 75.96) (width 0.5) (layer "F.Cu") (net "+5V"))
 (segment (start 185.54 75.96) (end 183 78.5) (width 0.5) (layer "F.Cu") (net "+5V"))
 (segment (start 175 75.525) (end 177.975 78.5) (width 0.5) (layer "F.Cu") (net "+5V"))
 (segment (start 226.726 63.283) (end 210.783 63.283) (width 0.4) (layer "F.Cu") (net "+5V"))
 (segment (start 191.08 75.5) (end 190.62 75.96) (width 0.5) (layer "F.Cu") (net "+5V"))
 (segment (start 209.5 62) (end 209.5 63.025) (width 0.4) (layer "F.Cu") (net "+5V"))
 (segment (start 195.525 77) (end 194.485 75.96) (width 0.4) (layer "F.Cu") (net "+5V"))
 (segment (start 183 78.5) (end 177.975 78.5) (width 0.5) (layer "F.Cu") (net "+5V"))
 (segment (start 209.5 63.025) (end 195.525 77) (width 0.4) (layer "F.Cu") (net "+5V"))
 (segment (start 210.783 63.283) (end 209.5 62) (width 0.4) (layer "F.Cu") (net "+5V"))
 (segment (start 175 71) (end 175 75.525) (width 0.5) (layer "F.Cu") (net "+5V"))
 (segment (start 194.485 75.96) (end 190.62 75.96) (width 0.4) (layer "F.Cu") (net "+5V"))
 (segment (start 183 68.34) (end 179.84 68.34) (width 0.5) (layer "F.Cu") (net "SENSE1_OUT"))
 (segment (start 179.84 68.34) (end 175 63.5) (width 0.5) (layer "F.Cu") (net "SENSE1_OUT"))
 (segment (start 190.62 70.461321) (end 190.62 70.88) (width 0.4) (layer "F.Cu") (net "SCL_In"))
 (segment (start 210.5 52) (end 208 52) (width 0.4) (layer "F.Cu") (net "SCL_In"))
 (segment (start 212 53.5) (end 210.5 52) (width 0.4) (layer "F.Cu") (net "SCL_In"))
 (segment (start 212 54.42) (end 212 53.5) (width 0.4) (layer "F.Cu") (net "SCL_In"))
 (segment (start 192.12 68.961321) (end 190.62 70.461321) (width 0.4) (layer "F.Cu") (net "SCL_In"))
 (segment (start 209.5 56.92) (end 212 54.42) (width 0.4) (layer "F.Cu") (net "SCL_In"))
 (segment (start 208 52) (end 192.12 67.88) (width 0.4) (layer "F.Cu") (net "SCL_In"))
 (segment (start 192.12 67.88) (end 192.12 68.961321) (width 0.4) (layer "F.Cu") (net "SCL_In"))
 (segment (start 209.5 54.38) (end 190.62 73.26) (width 0.4) (layer "F.Cu") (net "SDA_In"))
 (segment (start 190.62 73.26) (end 190.62 73.42) (width 0.4) (layer "F.Cu") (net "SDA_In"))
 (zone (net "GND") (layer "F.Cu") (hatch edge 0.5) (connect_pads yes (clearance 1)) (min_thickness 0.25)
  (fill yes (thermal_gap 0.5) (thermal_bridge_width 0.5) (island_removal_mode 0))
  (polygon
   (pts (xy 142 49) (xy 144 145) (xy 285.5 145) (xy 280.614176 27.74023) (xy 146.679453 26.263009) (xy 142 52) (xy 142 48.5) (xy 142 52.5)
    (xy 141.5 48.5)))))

